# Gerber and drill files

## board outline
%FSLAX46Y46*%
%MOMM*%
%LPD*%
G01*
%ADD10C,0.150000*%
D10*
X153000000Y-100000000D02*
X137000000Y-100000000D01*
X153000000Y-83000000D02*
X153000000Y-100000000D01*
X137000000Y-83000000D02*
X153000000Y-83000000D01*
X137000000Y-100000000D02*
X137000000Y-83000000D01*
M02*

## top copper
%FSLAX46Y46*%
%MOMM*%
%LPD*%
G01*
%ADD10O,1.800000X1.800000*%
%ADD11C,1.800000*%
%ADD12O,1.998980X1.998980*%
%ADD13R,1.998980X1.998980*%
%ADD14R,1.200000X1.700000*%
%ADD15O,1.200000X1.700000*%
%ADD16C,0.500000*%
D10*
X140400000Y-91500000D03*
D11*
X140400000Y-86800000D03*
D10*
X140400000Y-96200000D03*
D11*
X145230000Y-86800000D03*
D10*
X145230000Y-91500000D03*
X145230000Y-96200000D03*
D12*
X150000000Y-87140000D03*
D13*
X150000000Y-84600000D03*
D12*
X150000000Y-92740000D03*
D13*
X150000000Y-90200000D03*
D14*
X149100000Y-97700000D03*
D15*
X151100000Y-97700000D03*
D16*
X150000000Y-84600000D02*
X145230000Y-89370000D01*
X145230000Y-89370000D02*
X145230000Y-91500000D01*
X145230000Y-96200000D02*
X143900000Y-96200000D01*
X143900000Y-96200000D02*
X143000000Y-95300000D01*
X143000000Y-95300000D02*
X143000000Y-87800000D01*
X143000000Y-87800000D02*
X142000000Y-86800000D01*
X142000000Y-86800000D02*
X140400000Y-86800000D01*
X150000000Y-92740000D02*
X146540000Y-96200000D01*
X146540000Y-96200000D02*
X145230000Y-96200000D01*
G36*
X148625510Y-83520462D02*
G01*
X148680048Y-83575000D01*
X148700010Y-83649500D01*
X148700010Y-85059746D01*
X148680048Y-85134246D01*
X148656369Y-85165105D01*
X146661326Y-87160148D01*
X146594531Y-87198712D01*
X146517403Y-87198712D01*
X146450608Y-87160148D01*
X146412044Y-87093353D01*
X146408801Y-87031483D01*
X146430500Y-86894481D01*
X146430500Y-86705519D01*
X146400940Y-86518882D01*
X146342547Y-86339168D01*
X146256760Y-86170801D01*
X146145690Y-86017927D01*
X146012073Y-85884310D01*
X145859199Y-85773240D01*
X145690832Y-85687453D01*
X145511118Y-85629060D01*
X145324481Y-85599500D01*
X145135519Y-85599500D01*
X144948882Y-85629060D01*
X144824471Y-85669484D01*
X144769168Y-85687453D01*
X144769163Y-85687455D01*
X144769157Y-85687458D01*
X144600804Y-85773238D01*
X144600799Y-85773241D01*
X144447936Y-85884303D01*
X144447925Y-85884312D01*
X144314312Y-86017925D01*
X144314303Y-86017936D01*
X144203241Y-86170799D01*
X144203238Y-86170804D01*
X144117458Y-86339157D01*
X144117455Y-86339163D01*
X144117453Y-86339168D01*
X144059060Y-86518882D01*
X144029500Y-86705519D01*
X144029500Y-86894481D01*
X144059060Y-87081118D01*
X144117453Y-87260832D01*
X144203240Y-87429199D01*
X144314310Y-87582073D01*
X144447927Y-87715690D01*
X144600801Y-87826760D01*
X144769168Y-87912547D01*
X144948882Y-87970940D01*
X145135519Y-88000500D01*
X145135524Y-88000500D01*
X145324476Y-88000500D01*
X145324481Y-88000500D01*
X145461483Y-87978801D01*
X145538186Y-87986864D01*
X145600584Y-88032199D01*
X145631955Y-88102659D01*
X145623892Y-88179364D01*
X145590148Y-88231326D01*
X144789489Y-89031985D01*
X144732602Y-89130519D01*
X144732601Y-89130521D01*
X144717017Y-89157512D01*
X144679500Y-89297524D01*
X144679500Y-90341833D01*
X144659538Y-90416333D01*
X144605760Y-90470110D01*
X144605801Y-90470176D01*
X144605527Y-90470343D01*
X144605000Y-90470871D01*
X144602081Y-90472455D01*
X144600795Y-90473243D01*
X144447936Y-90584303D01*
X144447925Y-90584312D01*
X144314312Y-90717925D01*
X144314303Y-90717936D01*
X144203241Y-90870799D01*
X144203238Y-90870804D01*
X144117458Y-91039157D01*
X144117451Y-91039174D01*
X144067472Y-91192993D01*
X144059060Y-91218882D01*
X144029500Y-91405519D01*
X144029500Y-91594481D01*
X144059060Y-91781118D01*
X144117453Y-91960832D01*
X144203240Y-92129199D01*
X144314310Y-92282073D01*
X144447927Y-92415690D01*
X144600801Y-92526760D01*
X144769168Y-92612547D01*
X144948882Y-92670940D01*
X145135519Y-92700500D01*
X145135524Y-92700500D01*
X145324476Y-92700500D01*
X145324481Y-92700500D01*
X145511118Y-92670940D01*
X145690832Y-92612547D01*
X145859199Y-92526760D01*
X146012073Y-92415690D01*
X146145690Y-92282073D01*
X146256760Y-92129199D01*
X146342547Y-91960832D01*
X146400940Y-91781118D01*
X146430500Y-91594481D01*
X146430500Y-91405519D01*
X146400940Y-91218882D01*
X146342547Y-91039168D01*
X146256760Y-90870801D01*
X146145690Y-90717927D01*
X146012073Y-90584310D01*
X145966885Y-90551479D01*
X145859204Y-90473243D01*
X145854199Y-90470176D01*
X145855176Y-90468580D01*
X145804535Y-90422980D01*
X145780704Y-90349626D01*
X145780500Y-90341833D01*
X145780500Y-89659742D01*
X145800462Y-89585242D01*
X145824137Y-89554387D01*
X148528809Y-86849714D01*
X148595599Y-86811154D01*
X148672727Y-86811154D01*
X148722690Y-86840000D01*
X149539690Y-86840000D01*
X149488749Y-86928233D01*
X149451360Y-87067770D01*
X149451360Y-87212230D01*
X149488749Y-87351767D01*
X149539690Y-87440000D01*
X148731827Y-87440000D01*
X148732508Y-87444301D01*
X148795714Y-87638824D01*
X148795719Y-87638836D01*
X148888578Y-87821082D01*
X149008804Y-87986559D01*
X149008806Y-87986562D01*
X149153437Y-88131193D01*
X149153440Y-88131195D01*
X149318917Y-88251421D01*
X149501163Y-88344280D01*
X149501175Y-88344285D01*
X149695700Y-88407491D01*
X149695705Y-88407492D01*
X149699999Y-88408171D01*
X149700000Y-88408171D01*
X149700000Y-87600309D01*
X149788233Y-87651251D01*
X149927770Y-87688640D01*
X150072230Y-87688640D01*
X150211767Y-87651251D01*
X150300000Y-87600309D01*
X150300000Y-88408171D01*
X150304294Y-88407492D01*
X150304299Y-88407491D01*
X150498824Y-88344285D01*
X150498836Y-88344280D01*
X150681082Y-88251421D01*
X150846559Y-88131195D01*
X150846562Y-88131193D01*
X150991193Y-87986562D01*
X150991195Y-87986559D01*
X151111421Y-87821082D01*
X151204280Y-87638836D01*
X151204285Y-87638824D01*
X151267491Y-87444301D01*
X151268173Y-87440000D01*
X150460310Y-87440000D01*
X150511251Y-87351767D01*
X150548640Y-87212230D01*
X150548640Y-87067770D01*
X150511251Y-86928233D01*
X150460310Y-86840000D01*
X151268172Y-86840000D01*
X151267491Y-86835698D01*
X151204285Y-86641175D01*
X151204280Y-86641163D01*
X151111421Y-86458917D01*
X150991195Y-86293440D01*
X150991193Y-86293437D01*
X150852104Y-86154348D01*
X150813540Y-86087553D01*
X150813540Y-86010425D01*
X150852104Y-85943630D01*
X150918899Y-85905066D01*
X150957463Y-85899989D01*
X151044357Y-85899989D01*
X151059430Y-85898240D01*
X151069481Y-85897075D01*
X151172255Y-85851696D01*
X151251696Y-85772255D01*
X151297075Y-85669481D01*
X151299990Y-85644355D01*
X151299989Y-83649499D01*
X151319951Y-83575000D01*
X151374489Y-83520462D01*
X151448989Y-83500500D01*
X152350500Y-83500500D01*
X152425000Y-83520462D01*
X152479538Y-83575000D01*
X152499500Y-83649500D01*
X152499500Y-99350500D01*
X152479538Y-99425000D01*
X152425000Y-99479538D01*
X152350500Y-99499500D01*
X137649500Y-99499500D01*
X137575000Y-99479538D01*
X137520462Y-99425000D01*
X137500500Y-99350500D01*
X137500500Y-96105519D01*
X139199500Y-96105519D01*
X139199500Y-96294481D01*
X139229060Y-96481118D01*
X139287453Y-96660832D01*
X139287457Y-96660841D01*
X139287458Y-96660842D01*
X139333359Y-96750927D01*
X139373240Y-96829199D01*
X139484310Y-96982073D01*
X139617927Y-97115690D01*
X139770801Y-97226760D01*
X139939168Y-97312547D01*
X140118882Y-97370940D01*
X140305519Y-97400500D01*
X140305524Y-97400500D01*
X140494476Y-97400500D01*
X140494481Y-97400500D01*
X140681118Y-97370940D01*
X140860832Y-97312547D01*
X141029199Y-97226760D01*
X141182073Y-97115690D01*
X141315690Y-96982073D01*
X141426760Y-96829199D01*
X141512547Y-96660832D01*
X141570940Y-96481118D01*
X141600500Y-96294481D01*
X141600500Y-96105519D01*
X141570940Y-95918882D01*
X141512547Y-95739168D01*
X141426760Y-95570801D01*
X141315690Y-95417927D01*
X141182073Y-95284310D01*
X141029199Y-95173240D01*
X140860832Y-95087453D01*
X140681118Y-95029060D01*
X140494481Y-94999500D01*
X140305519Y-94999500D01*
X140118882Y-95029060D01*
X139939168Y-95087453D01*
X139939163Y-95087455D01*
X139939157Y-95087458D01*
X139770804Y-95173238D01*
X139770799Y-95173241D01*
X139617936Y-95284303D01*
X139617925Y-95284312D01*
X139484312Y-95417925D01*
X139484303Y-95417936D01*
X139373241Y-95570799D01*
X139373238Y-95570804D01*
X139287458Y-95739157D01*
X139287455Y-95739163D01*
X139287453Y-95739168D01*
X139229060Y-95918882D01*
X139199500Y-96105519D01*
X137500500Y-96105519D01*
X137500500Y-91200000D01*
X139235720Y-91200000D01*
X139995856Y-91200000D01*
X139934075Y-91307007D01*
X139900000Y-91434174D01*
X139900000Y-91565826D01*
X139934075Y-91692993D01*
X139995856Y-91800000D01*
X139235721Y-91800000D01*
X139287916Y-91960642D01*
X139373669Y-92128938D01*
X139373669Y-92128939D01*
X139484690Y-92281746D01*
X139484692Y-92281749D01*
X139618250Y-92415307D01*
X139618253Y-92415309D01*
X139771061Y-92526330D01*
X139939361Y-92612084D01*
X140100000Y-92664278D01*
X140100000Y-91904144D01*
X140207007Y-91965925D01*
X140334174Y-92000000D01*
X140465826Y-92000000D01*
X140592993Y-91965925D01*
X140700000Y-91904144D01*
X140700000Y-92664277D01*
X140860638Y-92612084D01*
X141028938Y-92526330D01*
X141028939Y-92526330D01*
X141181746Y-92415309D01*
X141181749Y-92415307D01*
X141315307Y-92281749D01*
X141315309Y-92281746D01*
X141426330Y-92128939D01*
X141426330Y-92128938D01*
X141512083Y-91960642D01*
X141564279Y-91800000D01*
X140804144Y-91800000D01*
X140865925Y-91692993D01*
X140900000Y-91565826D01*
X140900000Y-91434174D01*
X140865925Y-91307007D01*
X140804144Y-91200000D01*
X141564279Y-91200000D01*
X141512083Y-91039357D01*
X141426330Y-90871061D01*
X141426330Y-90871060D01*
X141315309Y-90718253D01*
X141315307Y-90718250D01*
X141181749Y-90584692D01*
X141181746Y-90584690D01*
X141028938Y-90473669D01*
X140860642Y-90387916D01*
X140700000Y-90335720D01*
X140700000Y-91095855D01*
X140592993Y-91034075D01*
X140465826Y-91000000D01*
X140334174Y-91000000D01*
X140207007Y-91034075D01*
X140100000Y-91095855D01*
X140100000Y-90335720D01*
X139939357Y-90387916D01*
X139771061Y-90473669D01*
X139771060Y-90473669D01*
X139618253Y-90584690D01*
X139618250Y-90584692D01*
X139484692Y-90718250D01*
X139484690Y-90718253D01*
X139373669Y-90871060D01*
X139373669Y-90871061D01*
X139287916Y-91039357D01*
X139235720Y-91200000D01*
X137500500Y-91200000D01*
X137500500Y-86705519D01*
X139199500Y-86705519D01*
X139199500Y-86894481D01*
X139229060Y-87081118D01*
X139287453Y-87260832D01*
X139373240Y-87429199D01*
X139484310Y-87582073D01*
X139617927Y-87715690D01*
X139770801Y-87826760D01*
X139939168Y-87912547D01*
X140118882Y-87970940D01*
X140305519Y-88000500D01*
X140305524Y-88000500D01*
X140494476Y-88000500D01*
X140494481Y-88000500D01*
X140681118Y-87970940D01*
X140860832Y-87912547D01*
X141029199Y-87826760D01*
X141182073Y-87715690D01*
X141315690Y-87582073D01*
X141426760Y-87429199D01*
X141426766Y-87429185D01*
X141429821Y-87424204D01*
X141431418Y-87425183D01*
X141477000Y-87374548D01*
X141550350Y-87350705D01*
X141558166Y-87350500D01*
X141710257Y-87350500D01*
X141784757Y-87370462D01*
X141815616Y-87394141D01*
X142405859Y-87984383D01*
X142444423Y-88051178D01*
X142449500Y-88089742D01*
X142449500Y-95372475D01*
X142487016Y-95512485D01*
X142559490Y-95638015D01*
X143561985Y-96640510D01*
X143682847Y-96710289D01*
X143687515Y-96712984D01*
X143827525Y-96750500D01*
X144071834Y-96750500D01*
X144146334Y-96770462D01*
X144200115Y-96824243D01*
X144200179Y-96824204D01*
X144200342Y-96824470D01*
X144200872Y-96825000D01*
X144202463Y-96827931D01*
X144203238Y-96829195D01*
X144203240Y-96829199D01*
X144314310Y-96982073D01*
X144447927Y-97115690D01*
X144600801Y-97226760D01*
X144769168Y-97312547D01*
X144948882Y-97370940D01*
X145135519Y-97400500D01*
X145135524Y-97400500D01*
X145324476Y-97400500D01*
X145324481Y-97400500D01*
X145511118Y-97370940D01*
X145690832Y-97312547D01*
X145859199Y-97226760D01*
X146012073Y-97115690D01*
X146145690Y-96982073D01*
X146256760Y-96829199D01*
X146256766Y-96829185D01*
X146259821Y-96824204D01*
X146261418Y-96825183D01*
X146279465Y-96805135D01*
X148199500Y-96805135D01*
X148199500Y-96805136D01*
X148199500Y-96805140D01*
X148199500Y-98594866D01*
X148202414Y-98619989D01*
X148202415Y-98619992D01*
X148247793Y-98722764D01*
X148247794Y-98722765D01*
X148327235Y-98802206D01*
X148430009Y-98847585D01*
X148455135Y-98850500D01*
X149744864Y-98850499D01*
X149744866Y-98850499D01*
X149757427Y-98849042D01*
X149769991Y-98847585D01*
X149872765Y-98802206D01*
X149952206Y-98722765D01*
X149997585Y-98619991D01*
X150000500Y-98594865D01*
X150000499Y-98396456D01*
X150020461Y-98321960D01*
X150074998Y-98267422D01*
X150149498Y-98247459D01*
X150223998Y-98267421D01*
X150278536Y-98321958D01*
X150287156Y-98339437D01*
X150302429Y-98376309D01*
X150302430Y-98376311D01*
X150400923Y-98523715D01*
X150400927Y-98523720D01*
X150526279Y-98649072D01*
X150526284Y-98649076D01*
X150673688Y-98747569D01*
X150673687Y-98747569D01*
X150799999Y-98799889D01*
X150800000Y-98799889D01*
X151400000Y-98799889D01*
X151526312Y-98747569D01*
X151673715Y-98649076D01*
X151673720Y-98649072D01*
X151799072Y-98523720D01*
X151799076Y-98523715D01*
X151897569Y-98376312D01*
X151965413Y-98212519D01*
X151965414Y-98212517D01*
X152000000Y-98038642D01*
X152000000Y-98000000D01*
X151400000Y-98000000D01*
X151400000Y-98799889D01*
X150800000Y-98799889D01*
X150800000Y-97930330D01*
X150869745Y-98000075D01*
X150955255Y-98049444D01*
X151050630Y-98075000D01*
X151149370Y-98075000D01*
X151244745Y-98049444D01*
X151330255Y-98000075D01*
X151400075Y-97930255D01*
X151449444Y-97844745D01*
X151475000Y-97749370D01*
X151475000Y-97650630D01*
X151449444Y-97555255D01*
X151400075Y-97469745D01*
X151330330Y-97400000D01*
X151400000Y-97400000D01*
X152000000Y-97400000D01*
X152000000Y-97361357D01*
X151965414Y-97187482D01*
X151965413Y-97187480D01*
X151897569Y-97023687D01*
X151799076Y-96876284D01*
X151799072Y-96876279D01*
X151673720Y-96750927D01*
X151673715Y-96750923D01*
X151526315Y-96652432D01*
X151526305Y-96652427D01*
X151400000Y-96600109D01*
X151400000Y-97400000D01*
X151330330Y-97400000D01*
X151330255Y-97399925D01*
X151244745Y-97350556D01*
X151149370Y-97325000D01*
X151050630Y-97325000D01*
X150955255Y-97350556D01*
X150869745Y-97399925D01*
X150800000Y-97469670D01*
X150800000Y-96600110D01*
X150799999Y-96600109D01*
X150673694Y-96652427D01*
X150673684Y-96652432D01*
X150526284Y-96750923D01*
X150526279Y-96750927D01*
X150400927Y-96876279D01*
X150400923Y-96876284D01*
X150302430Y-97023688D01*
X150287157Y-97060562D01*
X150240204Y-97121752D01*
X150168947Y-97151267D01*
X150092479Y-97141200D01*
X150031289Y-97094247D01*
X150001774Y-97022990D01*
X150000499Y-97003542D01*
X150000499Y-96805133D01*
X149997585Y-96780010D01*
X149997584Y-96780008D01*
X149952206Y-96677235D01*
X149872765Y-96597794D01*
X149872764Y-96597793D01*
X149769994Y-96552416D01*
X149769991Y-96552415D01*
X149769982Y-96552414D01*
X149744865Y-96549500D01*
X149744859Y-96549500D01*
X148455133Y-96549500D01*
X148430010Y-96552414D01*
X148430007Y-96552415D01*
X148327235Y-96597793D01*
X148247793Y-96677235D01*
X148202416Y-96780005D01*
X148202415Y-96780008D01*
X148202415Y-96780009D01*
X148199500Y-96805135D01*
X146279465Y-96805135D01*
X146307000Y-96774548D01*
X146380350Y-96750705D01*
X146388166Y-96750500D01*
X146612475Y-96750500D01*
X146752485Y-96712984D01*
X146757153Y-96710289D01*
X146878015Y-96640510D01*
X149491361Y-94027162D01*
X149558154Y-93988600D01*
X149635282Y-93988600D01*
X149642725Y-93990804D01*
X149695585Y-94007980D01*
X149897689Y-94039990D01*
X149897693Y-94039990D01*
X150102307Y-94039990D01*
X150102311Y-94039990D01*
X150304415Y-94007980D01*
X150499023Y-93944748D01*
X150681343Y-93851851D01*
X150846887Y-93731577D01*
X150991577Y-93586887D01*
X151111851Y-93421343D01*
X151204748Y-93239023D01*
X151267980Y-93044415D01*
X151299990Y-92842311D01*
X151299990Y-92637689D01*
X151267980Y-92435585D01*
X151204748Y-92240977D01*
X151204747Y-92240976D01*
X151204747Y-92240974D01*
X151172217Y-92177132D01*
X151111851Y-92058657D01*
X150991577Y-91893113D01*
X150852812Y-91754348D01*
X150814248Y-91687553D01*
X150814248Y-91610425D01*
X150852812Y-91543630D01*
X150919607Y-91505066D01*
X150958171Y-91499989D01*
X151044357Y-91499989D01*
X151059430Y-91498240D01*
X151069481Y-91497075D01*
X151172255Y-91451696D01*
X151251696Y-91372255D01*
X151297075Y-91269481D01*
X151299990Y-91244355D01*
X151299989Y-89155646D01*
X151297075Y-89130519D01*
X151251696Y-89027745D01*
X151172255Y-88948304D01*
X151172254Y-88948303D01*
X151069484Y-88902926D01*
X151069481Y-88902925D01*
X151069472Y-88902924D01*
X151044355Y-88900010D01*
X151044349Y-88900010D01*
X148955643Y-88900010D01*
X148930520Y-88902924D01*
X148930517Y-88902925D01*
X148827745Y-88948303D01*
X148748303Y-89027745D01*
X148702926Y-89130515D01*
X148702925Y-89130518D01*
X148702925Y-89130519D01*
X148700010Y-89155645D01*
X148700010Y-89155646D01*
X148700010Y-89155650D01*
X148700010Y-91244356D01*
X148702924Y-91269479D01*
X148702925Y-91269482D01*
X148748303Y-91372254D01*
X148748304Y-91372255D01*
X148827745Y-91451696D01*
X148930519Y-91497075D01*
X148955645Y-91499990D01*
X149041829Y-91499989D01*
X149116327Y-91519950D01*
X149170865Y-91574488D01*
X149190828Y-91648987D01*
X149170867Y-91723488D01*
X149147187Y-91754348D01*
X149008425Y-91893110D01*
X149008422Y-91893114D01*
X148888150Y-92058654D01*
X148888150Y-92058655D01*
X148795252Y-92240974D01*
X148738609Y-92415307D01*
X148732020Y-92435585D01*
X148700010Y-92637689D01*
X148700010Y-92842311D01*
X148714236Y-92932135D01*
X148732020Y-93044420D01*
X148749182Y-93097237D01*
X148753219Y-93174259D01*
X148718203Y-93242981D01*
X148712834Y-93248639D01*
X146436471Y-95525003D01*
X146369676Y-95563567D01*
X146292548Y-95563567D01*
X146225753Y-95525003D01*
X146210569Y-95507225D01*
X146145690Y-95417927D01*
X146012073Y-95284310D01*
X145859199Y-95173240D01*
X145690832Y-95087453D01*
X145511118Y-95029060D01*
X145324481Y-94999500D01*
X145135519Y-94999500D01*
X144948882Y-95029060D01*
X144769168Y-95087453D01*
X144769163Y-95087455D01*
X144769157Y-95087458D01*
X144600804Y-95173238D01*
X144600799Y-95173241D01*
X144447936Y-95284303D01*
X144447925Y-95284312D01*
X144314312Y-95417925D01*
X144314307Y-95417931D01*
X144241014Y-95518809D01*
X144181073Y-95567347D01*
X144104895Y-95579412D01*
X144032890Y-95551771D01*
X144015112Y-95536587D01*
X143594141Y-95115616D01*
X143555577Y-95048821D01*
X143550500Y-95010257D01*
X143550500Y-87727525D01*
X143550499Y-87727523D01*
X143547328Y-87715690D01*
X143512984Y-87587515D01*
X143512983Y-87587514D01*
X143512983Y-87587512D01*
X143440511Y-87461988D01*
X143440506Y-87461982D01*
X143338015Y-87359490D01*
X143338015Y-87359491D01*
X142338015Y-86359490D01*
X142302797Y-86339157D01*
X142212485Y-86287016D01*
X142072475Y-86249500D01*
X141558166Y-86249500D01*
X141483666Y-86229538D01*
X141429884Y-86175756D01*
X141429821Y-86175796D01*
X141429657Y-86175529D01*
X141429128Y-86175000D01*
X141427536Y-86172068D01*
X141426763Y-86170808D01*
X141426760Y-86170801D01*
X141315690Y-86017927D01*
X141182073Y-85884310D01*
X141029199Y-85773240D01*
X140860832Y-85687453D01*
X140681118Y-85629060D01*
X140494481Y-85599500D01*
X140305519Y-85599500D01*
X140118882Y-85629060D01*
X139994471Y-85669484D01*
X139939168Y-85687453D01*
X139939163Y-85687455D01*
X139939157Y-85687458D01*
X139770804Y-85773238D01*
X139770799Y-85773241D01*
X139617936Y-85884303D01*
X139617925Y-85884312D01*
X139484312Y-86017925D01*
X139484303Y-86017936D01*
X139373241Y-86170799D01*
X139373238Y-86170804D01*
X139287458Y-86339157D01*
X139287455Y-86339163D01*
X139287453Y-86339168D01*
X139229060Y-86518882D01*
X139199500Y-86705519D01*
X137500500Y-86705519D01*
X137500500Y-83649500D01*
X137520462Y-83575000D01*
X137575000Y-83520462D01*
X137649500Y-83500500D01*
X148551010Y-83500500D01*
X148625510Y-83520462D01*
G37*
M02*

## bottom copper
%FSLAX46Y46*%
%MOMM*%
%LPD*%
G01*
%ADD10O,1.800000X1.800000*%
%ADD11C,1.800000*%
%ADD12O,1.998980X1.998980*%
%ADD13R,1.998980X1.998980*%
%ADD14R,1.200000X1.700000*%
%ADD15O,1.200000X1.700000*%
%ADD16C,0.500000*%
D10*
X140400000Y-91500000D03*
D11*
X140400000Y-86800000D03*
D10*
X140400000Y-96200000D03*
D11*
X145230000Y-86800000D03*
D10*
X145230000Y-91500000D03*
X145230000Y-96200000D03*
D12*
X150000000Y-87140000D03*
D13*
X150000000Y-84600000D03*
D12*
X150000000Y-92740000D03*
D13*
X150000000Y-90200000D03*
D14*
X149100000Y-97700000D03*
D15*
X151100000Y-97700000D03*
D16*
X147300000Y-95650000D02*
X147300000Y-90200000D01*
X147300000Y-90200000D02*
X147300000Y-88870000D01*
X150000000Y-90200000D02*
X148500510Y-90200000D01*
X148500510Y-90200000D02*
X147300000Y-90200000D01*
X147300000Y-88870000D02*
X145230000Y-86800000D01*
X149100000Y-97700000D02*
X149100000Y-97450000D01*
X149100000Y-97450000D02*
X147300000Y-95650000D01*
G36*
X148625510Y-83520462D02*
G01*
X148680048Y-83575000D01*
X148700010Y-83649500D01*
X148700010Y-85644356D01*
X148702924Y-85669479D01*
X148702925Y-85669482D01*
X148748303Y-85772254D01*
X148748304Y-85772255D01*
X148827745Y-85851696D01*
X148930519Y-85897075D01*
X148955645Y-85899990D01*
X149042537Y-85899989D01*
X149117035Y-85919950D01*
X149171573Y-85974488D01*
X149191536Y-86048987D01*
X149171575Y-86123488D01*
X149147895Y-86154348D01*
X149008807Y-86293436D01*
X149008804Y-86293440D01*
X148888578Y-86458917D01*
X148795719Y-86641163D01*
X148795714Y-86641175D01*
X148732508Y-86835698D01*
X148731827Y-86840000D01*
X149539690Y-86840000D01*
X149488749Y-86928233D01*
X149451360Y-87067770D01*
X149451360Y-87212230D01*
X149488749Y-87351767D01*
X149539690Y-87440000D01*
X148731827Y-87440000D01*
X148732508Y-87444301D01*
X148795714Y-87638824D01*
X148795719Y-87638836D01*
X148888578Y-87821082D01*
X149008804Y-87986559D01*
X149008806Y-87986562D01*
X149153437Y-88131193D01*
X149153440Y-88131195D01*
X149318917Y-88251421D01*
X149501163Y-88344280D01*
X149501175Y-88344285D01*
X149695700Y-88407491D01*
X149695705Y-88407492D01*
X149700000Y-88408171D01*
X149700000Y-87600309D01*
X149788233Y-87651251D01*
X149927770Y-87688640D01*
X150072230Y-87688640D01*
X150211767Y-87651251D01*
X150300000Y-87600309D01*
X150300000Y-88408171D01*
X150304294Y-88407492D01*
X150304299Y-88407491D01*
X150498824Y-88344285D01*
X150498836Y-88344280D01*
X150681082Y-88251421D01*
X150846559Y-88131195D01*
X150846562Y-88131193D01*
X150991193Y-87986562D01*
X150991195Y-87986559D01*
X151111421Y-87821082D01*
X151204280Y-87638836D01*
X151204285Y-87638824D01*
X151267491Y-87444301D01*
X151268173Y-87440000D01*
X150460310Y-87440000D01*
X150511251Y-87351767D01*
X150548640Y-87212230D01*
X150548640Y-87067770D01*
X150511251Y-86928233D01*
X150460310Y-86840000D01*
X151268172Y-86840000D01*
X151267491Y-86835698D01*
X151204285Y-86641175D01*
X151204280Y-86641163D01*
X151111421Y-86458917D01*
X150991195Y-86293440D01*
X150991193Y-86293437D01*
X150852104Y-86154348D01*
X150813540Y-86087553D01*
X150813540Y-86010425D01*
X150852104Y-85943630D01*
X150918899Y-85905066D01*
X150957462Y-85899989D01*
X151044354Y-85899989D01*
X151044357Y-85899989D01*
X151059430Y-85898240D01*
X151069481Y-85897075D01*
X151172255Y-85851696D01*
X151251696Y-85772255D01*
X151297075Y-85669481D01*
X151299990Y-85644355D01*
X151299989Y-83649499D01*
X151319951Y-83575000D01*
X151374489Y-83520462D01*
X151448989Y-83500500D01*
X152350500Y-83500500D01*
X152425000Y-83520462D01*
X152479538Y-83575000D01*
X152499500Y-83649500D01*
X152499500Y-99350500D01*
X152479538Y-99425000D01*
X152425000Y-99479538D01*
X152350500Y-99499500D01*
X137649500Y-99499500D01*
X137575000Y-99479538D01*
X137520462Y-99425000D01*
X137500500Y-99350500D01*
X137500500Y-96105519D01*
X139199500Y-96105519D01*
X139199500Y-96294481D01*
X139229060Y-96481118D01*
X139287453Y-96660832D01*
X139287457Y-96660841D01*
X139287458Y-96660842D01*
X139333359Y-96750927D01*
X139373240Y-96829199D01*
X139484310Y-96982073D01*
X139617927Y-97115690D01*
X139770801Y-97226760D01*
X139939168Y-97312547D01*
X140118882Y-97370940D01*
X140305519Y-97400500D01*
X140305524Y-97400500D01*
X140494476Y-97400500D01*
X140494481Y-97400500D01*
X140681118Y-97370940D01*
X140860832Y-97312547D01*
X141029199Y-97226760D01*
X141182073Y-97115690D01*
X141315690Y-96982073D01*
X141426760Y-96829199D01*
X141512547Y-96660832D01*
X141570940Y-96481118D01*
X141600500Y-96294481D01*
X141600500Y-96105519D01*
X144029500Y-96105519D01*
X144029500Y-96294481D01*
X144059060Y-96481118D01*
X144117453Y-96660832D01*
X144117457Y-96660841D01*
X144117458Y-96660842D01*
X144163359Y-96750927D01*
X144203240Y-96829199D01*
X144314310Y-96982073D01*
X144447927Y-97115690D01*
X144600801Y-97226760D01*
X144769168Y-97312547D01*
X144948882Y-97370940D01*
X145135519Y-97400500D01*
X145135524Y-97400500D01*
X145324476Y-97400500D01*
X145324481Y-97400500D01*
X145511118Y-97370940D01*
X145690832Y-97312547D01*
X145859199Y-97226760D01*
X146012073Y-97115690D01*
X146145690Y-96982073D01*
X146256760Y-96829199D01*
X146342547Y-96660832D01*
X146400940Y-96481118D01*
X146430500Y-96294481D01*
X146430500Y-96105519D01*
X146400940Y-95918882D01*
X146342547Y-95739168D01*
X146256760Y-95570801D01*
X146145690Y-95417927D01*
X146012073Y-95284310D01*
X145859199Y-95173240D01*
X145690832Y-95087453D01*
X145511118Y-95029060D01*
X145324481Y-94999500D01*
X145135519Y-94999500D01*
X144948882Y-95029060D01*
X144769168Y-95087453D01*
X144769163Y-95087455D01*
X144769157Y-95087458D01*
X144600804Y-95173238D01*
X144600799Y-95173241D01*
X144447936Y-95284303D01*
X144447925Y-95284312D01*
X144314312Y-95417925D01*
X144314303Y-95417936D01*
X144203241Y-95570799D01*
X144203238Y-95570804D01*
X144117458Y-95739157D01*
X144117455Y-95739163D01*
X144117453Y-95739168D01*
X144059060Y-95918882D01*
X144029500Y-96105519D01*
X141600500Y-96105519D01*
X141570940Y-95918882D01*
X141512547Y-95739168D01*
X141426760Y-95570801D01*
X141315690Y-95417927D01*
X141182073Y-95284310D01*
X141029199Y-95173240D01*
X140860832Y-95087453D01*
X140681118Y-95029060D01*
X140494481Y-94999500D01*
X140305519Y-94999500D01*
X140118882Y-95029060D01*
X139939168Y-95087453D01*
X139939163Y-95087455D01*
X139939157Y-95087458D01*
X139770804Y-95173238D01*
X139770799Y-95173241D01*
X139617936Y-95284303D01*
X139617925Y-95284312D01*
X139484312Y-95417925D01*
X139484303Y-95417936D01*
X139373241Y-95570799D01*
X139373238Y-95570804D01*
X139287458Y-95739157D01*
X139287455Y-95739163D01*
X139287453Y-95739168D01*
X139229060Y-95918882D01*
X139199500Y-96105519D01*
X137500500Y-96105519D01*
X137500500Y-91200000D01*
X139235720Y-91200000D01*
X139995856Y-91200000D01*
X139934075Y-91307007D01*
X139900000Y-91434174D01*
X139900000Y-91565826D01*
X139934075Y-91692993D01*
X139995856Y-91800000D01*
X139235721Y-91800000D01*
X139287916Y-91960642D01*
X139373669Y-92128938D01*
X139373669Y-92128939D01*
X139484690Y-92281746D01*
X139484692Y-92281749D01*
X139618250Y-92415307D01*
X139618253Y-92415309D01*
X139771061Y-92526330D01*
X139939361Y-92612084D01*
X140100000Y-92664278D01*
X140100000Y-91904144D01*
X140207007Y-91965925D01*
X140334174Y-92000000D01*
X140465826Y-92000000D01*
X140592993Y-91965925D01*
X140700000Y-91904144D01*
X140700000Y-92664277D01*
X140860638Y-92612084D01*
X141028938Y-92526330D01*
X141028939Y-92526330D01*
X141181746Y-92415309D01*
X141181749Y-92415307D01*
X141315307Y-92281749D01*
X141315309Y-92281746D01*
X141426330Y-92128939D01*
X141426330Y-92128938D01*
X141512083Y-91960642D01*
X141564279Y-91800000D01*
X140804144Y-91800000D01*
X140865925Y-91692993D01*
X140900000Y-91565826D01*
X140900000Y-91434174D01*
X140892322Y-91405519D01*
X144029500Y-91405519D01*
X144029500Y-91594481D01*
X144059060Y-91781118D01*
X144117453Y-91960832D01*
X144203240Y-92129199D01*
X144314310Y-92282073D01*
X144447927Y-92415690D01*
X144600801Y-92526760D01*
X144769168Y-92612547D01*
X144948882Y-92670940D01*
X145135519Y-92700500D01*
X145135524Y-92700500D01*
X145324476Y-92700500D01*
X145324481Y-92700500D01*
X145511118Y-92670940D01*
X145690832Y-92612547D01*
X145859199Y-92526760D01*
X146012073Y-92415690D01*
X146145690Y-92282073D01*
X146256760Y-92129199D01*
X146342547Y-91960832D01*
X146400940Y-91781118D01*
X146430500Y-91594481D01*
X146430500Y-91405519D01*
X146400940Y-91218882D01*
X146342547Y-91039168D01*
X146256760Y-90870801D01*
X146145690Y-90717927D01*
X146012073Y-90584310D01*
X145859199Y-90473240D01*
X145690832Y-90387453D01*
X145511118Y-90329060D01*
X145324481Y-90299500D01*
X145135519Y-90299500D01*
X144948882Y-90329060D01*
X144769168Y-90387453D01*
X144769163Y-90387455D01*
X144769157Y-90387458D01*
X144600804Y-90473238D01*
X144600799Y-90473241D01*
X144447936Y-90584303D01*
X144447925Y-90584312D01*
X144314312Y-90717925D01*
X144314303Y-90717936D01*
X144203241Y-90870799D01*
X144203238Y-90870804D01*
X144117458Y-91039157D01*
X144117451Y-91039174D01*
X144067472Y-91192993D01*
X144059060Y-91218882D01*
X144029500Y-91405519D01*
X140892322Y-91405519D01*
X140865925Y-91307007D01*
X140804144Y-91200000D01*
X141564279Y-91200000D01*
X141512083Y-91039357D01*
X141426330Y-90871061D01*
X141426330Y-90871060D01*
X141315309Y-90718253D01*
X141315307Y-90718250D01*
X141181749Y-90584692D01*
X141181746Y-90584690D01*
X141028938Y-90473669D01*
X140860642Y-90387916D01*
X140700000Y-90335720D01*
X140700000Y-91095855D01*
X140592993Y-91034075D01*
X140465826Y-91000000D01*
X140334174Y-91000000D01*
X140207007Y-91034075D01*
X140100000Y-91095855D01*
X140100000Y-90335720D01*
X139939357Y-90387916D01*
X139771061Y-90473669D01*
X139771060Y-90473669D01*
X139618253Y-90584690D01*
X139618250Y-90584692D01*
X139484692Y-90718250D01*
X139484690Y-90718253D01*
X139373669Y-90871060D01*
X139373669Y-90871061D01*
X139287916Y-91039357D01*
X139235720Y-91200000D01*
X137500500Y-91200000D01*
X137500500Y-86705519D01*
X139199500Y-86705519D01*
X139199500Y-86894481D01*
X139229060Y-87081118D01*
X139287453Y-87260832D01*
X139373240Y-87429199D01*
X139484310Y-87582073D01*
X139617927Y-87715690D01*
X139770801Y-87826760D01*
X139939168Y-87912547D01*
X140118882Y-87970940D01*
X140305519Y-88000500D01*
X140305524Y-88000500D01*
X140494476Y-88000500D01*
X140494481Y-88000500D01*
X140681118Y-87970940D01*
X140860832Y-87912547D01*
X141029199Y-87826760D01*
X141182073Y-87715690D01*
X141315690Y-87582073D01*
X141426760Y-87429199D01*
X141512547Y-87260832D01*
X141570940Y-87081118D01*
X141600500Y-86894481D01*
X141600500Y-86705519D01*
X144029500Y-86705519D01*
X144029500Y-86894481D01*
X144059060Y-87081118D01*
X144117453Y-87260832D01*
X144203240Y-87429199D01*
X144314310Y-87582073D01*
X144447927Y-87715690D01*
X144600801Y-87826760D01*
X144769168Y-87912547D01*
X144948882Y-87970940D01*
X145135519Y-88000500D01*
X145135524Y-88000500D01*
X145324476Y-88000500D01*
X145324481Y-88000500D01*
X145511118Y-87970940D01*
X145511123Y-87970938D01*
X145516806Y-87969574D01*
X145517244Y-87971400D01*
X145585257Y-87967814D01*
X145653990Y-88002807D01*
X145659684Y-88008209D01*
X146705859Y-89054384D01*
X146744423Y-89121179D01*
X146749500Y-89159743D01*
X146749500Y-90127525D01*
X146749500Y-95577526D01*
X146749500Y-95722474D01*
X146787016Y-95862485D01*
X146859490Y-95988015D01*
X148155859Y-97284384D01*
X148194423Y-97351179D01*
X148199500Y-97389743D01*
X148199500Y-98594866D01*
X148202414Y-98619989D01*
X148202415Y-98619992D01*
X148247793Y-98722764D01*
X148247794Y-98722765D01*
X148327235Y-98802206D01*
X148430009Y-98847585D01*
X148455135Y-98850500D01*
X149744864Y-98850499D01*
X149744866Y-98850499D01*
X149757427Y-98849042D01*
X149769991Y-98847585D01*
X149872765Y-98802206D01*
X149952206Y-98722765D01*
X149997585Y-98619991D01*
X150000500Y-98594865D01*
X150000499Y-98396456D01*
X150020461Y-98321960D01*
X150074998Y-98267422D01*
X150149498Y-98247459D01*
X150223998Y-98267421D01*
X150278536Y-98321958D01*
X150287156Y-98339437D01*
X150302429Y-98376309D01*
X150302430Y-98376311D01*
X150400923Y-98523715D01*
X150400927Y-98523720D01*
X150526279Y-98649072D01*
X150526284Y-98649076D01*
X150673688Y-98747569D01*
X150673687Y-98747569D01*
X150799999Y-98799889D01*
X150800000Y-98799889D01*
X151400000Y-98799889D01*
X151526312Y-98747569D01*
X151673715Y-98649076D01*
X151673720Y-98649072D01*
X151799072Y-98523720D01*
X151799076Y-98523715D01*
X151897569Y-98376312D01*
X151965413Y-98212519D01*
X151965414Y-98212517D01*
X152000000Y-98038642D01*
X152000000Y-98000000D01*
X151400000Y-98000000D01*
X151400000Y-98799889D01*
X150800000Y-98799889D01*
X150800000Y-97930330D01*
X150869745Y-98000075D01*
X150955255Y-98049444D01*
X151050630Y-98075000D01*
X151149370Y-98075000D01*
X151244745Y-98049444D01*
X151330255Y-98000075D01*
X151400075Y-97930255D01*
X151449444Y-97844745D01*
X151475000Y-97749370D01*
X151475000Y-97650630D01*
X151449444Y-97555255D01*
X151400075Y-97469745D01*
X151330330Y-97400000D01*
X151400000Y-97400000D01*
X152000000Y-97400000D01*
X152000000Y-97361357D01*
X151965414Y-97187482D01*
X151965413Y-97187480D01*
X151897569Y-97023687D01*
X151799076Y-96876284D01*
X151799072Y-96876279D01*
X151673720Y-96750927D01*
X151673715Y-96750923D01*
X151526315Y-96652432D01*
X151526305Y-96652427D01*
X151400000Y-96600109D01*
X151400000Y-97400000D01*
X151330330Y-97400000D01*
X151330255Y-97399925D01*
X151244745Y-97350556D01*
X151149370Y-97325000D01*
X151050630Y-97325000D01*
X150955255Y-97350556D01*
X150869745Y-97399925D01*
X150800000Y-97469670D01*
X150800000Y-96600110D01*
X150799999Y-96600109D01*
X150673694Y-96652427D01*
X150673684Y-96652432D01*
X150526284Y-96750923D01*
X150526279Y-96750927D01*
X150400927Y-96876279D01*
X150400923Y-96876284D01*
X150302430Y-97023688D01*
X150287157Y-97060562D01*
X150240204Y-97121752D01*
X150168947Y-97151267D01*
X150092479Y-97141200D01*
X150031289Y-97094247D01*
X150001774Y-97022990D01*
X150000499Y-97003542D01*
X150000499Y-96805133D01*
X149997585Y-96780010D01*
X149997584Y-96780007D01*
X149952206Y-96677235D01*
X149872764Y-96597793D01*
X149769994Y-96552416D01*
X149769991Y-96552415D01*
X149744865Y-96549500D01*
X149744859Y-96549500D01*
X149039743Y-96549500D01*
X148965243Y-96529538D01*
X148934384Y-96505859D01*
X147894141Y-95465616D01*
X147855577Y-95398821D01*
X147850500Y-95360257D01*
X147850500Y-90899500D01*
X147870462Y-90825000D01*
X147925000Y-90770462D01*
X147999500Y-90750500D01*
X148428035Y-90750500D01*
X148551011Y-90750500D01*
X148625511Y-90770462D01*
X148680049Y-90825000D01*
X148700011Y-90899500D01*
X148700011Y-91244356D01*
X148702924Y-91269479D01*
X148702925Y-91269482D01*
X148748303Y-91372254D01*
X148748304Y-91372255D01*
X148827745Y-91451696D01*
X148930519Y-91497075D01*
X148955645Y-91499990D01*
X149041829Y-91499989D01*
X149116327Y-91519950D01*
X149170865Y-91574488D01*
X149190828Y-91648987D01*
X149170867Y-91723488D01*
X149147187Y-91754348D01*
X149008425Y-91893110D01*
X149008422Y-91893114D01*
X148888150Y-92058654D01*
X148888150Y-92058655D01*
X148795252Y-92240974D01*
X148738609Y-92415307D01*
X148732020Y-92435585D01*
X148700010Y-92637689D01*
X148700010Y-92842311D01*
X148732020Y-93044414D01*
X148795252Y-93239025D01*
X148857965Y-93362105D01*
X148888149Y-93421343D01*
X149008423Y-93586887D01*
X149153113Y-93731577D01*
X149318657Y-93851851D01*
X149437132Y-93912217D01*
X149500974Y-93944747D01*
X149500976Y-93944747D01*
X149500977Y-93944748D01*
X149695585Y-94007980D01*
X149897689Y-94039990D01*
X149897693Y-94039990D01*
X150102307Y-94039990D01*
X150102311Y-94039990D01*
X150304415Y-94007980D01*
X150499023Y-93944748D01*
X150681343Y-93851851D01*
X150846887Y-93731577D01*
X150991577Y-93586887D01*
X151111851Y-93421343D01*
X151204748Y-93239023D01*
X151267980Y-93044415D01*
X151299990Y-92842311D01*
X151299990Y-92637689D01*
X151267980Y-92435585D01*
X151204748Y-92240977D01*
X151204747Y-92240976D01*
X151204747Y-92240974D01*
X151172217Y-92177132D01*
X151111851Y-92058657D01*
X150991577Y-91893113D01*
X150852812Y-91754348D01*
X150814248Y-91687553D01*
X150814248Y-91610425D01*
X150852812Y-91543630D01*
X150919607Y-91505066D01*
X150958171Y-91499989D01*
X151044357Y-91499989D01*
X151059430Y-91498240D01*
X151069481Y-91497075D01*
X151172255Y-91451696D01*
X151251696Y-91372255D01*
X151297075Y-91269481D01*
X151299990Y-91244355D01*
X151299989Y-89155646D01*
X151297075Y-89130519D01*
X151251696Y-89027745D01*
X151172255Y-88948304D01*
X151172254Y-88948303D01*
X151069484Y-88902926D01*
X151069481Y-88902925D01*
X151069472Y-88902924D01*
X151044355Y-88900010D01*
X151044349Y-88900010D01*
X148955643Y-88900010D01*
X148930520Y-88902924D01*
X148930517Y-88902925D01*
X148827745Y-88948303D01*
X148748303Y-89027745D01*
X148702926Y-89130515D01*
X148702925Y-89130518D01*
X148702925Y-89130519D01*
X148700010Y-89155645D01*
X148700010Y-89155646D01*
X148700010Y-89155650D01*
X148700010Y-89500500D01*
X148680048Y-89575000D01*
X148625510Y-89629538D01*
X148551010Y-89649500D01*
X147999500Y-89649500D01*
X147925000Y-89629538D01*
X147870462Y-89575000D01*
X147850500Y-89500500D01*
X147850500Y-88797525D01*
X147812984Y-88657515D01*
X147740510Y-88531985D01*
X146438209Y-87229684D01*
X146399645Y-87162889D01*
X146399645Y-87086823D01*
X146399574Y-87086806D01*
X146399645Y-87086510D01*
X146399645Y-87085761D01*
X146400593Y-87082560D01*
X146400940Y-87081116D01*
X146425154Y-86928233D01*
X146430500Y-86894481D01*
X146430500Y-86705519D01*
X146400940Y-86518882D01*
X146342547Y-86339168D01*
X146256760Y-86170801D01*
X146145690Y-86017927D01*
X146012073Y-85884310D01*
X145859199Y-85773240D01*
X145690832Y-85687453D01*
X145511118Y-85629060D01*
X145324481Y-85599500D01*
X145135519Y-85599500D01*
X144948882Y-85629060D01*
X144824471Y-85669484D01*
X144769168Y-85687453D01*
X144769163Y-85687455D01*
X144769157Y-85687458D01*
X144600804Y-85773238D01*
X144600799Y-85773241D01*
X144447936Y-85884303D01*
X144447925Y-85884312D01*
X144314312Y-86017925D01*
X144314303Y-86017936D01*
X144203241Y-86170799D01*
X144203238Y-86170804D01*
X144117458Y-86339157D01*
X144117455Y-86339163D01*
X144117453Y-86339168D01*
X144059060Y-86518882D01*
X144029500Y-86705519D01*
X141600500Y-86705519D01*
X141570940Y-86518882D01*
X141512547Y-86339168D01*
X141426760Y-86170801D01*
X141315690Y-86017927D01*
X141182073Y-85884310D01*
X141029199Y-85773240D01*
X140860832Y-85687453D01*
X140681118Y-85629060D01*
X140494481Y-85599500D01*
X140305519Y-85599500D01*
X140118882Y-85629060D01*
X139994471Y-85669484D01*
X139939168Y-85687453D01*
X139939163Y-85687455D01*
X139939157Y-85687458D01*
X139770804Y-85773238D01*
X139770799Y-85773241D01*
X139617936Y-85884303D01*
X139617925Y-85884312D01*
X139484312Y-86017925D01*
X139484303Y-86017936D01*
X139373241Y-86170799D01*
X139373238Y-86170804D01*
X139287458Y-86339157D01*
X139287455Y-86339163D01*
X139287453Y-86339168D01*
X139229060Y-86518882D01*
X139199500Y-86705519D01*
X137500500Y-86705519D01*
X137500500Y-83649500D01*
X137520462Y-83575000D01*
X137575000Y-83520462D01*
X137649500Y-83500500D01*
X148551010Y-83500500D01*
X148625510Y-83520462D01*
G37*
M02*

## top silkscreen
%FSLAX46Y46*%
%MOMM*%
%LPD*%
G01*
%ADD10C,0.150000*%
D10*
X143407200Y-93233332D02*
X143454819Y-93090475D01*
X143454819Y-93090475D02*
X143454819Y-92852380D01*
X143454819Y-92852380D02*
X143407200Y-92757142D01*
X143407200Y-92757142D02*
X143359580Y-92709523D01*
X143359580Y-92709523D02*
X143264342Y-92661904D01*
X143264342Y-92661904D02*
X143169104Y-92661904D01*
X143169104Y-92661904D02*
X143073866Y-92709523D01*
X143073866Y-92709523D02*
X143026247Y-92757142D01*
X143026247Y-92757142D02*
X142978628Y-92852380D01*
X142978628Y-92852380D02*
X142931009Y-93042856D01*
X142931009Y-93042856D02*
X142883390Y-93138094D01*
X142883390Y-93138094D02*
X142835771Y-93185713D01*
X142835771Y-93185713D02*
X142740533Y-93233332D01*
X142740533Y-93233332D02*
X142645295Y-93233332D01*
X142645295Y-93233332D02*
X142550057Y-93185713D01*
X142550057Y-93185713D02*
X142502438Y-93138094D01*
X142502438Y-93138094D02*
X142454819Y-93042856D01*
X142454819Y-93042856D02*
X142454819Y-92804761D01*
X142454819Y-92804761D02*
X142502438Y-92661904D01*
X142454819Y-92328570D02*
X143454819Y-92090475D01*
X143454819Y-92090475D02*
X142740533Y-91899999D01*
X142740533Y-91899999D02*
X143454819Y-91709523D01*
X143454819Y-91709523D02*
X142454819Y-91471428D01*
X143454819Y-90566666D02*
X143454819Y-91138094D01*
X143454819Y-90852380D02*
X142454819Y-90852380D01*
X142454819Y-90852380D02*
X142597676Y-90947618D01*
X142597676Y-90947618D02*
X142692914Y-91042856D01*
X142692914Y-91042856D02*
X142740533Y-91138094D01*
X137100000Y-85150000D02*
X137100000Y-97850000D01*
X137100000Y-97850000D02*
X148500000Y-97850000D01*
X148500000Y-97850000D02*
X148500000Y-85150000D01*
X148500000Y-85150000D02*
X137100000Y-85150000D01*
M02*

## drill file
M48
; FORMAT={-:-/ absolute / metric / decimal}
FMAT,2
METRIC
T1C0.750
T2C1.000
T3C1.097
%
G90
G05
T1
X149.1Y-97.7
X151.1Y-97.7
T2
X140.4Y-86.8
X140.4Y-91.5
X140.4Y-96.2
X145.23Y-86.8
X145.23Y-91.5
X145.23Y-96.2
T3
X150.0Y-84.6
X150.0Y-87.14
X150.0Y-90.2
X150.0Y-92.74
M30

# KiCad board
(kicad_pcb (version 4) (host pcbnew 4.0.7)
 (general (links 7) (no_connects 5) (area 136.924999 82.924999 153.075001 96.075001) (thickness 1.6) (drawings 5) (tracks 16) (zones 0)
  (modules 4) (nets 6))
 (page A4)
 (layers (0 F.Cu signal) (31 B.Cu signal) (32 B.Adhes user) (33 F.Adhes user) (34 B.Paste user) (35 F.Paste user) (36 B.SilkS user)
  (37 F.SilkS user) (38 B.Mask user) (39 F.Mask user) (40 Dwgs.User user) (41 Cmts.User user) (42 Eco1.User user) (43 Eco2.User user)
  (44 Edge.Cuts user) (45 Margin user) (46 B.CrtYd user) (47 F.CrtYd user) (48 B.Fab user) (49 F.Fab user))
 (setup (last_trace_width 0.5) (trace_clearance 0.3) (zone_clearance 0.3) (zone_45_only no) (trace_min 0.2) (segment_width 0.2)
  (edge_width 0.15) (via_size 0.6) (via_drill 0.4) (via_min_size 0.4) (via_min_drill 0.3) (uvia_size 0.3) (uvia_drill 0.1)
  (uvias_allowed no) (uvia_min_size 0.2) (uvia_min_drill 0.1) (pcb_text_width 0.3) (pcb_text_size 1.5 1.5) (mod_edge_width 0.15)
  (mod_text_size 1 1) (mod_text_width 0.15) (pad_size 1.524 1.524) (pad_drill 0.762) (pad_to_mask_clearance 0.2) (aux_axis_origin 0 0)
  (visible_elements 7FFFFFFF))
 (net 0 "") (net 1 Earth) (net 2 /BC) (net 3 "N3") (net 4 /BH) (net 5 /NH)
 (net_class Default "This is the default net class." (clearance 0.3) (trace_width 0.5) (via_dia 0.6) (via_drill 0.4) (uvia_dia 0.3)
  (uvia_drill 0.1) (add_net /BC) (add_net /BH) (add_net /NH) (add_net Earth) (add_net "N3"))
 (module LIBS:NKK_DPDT (layer F.Cu) (at 145.2 86.8 90)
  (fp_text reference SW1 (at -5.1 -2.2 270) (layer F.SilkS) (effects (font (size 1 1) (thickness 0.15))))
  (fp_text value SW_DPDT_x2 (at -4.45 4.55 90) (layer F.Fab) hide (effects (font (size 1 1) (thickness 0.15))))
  (fp_line (start 1.65 -8.1) (end -11.05 -8.1) (layer F.SilkS) (width 0.15))
  (fp_line (start -11.05 -8.1) (end -11.05 3.3) (layer F.SilkS) (width 0.15))
  (fp_line (start -11.05 3.3) (end 1.65 3.3) (layer F.SilkS) (width 0.15))
  (fp_line (start 1.65 3.3) (end 1.65 -8.1) (layer F.SilkS) (width 0.15))
  (pad 5 thru_hole oval (at -4.7 -4.8 270) (size 1.8 1.8) (drill 1) (layers *.Cu *.Mask) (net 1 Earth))
  (pad 4 thru_hole circle (at 0 -4.8 270) (size 1.8 1.8) (drill 1) (layers *.Cu *.Mask) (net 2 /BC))
  (pad 6 thru_hole oval (at -9.4 -4.8 270) (size 1.8 1.8) (drill 1) (layers *.Cu *.Mask) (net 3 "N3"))
  (pad 1 thru_hole circle (at 0 0.03 270) (size 1.8 1.8) (drill 1) (layers *.Cu *.Mask) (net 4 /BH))
  (pad 2 thru_hole oval (at -4.7 0.03 270) (size 1.8 1.8) (drill 1) (layers *.Cu *.Mask) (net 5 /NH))
  (pad 3 thru_hole oval (at -9.4 0.03 270) (size 1.8 1.8) (drill 1) (layers *.Cu *.Mask) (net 2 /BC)))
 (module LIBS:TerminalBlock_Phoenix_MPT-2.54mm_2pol (layer B.Cu) (at 150 84.6 270)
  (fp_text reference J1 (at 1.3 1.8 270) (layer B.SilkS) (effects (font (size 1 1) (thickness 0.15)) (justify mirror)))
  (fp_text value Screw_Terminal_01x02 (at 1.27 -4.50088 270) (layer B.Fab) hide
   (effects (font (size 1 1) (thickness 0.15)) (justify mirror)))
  (pad 2 thru_hole oval (at 2.54 0 270) (size 1.99898 1.99898) (drill 1.09728) (layers *.Cu *.Mask) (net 1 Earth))
  (pad 1 thru_hole rect (at 0 0 270) (size 1.99898 1.99898) (drill 1.09728) (layers *.Cu *.Mask) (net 5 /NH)))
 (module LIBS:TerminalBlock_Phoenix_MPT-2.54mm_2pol (layer B.Cu) (at 150 90.2 270)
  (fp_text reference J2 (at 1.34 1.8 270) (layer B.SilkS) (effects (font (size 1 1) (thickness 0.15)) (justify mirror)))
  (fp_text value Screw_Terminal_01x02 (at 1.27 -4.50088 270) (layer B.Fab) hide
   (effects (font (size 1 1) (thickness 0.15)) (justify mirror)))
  (pad 2 thru_hole oval (at 2.54 0 270) (size 1.99898 1.99898) (drill 1.09728) (layers *.Cu *.Mask) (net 2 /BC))
  (pad 1 thru_hole rect (at 0 0 270) (size 1.99898 1.99898) (drill 1.09728) (layers *.Cu *.Mask) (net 4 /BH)))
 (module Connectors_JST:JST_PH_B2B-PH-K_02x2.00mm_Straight (layer B.Cu) (at 149.1 97.7)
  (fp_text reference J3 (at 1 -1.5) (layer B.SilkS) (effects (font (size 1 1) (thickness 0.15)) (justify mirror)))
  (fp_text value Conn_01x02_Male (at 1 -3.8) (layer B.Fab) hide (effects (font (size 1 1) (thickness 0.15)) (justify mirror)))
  (pad 1 thru_hole rect (at 0 0) (size 1.2 1.7) (drill 0.75) (layers *.Cu *.Mask) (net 4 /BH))
  (pad 2 thru_hole oval (at 2 0) (size 1.2 1.7) (drill 0.75) (layers *.Cu *.Mask) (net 1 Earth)))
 (gr_line (start 153 100) (end 137 100) (layer Edge.Cuts) (width 0.15))
 (gr_line (start 153 83) (end 153 100) (layer Edge.Cuts) (width 0.15))
 (gr_line (start 137 83) (end 153 83) (layer Edge.Cuts) (width 0.15))
 (gr_line (start 137 100) (end 137 83) (layer Edge.Cuts) (width 0.15))
 (segment (start 150 84.6) (end 145.23 89.37) (width 0.5) (layer F.Cu) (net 5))
 (segment (start 145.23 89.37) (end 145.23 91.5) (width 0.5) (layer F.Cu) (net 5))
 (segment (start 145.23 96.2) (end 143.9 96.2) (width 0.5) (layer F.Cu) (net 2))
 (segment (start 143.9 96.2) (end 143 95.3) (width 0.5) (layer F.Cu) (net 2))
 (segment (start 143 95.3) (end 143 87.8) (width 0.5) (layer F.Cu) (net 2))
 (segment (start 143 87.8) (end 142 86.8) (width 0.5) (layer F.Cu) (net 2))
 (segment (start 142 86.8) (end 140.4 86.8) (width 0.5) (layer F.Cu) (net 2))
 (segment (start 150 92.74) (end 146.54 96.2) (width 0.5) (layer F.Cu) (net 2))
 (segment (start 146.54 96.2) (end 145.23 96.2) (width 0.5) (layer F.Cu) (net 2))
 (segment (start 147.3 95.65) (end 147.3 90.2) (width 0.5) (layer B.Cu) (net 4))
 (segment (start 147.3 90.2) (end 147.3 88.87) (width 0.5) (layer B.Cu) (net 4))
 (segment (start 150 90.2) (end 148.50051 90.2) (width 0.5) (layer B.Cu) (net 4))
 (segment (start 148.50051 90.2) (end 147.3 90.2) (width 0.5) (layer B.Cu) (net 4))
 (segment (start 147.3 88.87) (end 145.23 86.8) (width 0.5) (layer B.Cu) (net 4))
 (segment (start 149.1 97.7) (end 149.1 97.45) (width 0.5) (layer B.Cu) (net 4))
 (segment (start 149.1 97.45) (end 147.3 95.65) (width 0.5) (layer B.Cu) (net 4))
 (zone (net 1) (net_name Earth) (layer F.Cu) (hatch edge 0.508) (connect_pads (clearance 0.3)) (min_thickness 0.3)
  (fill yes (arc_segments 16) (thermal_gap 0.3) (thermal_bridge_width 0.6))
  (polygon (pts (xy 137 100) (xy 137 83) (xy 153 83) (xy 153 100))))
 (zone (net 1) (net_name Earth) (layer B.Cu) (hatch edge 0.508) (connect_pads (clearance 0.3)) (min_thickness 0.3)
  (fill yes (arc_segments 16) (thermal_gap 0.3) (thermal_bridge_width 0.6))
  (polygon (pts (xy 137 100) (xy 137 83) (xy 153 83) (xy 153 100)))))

